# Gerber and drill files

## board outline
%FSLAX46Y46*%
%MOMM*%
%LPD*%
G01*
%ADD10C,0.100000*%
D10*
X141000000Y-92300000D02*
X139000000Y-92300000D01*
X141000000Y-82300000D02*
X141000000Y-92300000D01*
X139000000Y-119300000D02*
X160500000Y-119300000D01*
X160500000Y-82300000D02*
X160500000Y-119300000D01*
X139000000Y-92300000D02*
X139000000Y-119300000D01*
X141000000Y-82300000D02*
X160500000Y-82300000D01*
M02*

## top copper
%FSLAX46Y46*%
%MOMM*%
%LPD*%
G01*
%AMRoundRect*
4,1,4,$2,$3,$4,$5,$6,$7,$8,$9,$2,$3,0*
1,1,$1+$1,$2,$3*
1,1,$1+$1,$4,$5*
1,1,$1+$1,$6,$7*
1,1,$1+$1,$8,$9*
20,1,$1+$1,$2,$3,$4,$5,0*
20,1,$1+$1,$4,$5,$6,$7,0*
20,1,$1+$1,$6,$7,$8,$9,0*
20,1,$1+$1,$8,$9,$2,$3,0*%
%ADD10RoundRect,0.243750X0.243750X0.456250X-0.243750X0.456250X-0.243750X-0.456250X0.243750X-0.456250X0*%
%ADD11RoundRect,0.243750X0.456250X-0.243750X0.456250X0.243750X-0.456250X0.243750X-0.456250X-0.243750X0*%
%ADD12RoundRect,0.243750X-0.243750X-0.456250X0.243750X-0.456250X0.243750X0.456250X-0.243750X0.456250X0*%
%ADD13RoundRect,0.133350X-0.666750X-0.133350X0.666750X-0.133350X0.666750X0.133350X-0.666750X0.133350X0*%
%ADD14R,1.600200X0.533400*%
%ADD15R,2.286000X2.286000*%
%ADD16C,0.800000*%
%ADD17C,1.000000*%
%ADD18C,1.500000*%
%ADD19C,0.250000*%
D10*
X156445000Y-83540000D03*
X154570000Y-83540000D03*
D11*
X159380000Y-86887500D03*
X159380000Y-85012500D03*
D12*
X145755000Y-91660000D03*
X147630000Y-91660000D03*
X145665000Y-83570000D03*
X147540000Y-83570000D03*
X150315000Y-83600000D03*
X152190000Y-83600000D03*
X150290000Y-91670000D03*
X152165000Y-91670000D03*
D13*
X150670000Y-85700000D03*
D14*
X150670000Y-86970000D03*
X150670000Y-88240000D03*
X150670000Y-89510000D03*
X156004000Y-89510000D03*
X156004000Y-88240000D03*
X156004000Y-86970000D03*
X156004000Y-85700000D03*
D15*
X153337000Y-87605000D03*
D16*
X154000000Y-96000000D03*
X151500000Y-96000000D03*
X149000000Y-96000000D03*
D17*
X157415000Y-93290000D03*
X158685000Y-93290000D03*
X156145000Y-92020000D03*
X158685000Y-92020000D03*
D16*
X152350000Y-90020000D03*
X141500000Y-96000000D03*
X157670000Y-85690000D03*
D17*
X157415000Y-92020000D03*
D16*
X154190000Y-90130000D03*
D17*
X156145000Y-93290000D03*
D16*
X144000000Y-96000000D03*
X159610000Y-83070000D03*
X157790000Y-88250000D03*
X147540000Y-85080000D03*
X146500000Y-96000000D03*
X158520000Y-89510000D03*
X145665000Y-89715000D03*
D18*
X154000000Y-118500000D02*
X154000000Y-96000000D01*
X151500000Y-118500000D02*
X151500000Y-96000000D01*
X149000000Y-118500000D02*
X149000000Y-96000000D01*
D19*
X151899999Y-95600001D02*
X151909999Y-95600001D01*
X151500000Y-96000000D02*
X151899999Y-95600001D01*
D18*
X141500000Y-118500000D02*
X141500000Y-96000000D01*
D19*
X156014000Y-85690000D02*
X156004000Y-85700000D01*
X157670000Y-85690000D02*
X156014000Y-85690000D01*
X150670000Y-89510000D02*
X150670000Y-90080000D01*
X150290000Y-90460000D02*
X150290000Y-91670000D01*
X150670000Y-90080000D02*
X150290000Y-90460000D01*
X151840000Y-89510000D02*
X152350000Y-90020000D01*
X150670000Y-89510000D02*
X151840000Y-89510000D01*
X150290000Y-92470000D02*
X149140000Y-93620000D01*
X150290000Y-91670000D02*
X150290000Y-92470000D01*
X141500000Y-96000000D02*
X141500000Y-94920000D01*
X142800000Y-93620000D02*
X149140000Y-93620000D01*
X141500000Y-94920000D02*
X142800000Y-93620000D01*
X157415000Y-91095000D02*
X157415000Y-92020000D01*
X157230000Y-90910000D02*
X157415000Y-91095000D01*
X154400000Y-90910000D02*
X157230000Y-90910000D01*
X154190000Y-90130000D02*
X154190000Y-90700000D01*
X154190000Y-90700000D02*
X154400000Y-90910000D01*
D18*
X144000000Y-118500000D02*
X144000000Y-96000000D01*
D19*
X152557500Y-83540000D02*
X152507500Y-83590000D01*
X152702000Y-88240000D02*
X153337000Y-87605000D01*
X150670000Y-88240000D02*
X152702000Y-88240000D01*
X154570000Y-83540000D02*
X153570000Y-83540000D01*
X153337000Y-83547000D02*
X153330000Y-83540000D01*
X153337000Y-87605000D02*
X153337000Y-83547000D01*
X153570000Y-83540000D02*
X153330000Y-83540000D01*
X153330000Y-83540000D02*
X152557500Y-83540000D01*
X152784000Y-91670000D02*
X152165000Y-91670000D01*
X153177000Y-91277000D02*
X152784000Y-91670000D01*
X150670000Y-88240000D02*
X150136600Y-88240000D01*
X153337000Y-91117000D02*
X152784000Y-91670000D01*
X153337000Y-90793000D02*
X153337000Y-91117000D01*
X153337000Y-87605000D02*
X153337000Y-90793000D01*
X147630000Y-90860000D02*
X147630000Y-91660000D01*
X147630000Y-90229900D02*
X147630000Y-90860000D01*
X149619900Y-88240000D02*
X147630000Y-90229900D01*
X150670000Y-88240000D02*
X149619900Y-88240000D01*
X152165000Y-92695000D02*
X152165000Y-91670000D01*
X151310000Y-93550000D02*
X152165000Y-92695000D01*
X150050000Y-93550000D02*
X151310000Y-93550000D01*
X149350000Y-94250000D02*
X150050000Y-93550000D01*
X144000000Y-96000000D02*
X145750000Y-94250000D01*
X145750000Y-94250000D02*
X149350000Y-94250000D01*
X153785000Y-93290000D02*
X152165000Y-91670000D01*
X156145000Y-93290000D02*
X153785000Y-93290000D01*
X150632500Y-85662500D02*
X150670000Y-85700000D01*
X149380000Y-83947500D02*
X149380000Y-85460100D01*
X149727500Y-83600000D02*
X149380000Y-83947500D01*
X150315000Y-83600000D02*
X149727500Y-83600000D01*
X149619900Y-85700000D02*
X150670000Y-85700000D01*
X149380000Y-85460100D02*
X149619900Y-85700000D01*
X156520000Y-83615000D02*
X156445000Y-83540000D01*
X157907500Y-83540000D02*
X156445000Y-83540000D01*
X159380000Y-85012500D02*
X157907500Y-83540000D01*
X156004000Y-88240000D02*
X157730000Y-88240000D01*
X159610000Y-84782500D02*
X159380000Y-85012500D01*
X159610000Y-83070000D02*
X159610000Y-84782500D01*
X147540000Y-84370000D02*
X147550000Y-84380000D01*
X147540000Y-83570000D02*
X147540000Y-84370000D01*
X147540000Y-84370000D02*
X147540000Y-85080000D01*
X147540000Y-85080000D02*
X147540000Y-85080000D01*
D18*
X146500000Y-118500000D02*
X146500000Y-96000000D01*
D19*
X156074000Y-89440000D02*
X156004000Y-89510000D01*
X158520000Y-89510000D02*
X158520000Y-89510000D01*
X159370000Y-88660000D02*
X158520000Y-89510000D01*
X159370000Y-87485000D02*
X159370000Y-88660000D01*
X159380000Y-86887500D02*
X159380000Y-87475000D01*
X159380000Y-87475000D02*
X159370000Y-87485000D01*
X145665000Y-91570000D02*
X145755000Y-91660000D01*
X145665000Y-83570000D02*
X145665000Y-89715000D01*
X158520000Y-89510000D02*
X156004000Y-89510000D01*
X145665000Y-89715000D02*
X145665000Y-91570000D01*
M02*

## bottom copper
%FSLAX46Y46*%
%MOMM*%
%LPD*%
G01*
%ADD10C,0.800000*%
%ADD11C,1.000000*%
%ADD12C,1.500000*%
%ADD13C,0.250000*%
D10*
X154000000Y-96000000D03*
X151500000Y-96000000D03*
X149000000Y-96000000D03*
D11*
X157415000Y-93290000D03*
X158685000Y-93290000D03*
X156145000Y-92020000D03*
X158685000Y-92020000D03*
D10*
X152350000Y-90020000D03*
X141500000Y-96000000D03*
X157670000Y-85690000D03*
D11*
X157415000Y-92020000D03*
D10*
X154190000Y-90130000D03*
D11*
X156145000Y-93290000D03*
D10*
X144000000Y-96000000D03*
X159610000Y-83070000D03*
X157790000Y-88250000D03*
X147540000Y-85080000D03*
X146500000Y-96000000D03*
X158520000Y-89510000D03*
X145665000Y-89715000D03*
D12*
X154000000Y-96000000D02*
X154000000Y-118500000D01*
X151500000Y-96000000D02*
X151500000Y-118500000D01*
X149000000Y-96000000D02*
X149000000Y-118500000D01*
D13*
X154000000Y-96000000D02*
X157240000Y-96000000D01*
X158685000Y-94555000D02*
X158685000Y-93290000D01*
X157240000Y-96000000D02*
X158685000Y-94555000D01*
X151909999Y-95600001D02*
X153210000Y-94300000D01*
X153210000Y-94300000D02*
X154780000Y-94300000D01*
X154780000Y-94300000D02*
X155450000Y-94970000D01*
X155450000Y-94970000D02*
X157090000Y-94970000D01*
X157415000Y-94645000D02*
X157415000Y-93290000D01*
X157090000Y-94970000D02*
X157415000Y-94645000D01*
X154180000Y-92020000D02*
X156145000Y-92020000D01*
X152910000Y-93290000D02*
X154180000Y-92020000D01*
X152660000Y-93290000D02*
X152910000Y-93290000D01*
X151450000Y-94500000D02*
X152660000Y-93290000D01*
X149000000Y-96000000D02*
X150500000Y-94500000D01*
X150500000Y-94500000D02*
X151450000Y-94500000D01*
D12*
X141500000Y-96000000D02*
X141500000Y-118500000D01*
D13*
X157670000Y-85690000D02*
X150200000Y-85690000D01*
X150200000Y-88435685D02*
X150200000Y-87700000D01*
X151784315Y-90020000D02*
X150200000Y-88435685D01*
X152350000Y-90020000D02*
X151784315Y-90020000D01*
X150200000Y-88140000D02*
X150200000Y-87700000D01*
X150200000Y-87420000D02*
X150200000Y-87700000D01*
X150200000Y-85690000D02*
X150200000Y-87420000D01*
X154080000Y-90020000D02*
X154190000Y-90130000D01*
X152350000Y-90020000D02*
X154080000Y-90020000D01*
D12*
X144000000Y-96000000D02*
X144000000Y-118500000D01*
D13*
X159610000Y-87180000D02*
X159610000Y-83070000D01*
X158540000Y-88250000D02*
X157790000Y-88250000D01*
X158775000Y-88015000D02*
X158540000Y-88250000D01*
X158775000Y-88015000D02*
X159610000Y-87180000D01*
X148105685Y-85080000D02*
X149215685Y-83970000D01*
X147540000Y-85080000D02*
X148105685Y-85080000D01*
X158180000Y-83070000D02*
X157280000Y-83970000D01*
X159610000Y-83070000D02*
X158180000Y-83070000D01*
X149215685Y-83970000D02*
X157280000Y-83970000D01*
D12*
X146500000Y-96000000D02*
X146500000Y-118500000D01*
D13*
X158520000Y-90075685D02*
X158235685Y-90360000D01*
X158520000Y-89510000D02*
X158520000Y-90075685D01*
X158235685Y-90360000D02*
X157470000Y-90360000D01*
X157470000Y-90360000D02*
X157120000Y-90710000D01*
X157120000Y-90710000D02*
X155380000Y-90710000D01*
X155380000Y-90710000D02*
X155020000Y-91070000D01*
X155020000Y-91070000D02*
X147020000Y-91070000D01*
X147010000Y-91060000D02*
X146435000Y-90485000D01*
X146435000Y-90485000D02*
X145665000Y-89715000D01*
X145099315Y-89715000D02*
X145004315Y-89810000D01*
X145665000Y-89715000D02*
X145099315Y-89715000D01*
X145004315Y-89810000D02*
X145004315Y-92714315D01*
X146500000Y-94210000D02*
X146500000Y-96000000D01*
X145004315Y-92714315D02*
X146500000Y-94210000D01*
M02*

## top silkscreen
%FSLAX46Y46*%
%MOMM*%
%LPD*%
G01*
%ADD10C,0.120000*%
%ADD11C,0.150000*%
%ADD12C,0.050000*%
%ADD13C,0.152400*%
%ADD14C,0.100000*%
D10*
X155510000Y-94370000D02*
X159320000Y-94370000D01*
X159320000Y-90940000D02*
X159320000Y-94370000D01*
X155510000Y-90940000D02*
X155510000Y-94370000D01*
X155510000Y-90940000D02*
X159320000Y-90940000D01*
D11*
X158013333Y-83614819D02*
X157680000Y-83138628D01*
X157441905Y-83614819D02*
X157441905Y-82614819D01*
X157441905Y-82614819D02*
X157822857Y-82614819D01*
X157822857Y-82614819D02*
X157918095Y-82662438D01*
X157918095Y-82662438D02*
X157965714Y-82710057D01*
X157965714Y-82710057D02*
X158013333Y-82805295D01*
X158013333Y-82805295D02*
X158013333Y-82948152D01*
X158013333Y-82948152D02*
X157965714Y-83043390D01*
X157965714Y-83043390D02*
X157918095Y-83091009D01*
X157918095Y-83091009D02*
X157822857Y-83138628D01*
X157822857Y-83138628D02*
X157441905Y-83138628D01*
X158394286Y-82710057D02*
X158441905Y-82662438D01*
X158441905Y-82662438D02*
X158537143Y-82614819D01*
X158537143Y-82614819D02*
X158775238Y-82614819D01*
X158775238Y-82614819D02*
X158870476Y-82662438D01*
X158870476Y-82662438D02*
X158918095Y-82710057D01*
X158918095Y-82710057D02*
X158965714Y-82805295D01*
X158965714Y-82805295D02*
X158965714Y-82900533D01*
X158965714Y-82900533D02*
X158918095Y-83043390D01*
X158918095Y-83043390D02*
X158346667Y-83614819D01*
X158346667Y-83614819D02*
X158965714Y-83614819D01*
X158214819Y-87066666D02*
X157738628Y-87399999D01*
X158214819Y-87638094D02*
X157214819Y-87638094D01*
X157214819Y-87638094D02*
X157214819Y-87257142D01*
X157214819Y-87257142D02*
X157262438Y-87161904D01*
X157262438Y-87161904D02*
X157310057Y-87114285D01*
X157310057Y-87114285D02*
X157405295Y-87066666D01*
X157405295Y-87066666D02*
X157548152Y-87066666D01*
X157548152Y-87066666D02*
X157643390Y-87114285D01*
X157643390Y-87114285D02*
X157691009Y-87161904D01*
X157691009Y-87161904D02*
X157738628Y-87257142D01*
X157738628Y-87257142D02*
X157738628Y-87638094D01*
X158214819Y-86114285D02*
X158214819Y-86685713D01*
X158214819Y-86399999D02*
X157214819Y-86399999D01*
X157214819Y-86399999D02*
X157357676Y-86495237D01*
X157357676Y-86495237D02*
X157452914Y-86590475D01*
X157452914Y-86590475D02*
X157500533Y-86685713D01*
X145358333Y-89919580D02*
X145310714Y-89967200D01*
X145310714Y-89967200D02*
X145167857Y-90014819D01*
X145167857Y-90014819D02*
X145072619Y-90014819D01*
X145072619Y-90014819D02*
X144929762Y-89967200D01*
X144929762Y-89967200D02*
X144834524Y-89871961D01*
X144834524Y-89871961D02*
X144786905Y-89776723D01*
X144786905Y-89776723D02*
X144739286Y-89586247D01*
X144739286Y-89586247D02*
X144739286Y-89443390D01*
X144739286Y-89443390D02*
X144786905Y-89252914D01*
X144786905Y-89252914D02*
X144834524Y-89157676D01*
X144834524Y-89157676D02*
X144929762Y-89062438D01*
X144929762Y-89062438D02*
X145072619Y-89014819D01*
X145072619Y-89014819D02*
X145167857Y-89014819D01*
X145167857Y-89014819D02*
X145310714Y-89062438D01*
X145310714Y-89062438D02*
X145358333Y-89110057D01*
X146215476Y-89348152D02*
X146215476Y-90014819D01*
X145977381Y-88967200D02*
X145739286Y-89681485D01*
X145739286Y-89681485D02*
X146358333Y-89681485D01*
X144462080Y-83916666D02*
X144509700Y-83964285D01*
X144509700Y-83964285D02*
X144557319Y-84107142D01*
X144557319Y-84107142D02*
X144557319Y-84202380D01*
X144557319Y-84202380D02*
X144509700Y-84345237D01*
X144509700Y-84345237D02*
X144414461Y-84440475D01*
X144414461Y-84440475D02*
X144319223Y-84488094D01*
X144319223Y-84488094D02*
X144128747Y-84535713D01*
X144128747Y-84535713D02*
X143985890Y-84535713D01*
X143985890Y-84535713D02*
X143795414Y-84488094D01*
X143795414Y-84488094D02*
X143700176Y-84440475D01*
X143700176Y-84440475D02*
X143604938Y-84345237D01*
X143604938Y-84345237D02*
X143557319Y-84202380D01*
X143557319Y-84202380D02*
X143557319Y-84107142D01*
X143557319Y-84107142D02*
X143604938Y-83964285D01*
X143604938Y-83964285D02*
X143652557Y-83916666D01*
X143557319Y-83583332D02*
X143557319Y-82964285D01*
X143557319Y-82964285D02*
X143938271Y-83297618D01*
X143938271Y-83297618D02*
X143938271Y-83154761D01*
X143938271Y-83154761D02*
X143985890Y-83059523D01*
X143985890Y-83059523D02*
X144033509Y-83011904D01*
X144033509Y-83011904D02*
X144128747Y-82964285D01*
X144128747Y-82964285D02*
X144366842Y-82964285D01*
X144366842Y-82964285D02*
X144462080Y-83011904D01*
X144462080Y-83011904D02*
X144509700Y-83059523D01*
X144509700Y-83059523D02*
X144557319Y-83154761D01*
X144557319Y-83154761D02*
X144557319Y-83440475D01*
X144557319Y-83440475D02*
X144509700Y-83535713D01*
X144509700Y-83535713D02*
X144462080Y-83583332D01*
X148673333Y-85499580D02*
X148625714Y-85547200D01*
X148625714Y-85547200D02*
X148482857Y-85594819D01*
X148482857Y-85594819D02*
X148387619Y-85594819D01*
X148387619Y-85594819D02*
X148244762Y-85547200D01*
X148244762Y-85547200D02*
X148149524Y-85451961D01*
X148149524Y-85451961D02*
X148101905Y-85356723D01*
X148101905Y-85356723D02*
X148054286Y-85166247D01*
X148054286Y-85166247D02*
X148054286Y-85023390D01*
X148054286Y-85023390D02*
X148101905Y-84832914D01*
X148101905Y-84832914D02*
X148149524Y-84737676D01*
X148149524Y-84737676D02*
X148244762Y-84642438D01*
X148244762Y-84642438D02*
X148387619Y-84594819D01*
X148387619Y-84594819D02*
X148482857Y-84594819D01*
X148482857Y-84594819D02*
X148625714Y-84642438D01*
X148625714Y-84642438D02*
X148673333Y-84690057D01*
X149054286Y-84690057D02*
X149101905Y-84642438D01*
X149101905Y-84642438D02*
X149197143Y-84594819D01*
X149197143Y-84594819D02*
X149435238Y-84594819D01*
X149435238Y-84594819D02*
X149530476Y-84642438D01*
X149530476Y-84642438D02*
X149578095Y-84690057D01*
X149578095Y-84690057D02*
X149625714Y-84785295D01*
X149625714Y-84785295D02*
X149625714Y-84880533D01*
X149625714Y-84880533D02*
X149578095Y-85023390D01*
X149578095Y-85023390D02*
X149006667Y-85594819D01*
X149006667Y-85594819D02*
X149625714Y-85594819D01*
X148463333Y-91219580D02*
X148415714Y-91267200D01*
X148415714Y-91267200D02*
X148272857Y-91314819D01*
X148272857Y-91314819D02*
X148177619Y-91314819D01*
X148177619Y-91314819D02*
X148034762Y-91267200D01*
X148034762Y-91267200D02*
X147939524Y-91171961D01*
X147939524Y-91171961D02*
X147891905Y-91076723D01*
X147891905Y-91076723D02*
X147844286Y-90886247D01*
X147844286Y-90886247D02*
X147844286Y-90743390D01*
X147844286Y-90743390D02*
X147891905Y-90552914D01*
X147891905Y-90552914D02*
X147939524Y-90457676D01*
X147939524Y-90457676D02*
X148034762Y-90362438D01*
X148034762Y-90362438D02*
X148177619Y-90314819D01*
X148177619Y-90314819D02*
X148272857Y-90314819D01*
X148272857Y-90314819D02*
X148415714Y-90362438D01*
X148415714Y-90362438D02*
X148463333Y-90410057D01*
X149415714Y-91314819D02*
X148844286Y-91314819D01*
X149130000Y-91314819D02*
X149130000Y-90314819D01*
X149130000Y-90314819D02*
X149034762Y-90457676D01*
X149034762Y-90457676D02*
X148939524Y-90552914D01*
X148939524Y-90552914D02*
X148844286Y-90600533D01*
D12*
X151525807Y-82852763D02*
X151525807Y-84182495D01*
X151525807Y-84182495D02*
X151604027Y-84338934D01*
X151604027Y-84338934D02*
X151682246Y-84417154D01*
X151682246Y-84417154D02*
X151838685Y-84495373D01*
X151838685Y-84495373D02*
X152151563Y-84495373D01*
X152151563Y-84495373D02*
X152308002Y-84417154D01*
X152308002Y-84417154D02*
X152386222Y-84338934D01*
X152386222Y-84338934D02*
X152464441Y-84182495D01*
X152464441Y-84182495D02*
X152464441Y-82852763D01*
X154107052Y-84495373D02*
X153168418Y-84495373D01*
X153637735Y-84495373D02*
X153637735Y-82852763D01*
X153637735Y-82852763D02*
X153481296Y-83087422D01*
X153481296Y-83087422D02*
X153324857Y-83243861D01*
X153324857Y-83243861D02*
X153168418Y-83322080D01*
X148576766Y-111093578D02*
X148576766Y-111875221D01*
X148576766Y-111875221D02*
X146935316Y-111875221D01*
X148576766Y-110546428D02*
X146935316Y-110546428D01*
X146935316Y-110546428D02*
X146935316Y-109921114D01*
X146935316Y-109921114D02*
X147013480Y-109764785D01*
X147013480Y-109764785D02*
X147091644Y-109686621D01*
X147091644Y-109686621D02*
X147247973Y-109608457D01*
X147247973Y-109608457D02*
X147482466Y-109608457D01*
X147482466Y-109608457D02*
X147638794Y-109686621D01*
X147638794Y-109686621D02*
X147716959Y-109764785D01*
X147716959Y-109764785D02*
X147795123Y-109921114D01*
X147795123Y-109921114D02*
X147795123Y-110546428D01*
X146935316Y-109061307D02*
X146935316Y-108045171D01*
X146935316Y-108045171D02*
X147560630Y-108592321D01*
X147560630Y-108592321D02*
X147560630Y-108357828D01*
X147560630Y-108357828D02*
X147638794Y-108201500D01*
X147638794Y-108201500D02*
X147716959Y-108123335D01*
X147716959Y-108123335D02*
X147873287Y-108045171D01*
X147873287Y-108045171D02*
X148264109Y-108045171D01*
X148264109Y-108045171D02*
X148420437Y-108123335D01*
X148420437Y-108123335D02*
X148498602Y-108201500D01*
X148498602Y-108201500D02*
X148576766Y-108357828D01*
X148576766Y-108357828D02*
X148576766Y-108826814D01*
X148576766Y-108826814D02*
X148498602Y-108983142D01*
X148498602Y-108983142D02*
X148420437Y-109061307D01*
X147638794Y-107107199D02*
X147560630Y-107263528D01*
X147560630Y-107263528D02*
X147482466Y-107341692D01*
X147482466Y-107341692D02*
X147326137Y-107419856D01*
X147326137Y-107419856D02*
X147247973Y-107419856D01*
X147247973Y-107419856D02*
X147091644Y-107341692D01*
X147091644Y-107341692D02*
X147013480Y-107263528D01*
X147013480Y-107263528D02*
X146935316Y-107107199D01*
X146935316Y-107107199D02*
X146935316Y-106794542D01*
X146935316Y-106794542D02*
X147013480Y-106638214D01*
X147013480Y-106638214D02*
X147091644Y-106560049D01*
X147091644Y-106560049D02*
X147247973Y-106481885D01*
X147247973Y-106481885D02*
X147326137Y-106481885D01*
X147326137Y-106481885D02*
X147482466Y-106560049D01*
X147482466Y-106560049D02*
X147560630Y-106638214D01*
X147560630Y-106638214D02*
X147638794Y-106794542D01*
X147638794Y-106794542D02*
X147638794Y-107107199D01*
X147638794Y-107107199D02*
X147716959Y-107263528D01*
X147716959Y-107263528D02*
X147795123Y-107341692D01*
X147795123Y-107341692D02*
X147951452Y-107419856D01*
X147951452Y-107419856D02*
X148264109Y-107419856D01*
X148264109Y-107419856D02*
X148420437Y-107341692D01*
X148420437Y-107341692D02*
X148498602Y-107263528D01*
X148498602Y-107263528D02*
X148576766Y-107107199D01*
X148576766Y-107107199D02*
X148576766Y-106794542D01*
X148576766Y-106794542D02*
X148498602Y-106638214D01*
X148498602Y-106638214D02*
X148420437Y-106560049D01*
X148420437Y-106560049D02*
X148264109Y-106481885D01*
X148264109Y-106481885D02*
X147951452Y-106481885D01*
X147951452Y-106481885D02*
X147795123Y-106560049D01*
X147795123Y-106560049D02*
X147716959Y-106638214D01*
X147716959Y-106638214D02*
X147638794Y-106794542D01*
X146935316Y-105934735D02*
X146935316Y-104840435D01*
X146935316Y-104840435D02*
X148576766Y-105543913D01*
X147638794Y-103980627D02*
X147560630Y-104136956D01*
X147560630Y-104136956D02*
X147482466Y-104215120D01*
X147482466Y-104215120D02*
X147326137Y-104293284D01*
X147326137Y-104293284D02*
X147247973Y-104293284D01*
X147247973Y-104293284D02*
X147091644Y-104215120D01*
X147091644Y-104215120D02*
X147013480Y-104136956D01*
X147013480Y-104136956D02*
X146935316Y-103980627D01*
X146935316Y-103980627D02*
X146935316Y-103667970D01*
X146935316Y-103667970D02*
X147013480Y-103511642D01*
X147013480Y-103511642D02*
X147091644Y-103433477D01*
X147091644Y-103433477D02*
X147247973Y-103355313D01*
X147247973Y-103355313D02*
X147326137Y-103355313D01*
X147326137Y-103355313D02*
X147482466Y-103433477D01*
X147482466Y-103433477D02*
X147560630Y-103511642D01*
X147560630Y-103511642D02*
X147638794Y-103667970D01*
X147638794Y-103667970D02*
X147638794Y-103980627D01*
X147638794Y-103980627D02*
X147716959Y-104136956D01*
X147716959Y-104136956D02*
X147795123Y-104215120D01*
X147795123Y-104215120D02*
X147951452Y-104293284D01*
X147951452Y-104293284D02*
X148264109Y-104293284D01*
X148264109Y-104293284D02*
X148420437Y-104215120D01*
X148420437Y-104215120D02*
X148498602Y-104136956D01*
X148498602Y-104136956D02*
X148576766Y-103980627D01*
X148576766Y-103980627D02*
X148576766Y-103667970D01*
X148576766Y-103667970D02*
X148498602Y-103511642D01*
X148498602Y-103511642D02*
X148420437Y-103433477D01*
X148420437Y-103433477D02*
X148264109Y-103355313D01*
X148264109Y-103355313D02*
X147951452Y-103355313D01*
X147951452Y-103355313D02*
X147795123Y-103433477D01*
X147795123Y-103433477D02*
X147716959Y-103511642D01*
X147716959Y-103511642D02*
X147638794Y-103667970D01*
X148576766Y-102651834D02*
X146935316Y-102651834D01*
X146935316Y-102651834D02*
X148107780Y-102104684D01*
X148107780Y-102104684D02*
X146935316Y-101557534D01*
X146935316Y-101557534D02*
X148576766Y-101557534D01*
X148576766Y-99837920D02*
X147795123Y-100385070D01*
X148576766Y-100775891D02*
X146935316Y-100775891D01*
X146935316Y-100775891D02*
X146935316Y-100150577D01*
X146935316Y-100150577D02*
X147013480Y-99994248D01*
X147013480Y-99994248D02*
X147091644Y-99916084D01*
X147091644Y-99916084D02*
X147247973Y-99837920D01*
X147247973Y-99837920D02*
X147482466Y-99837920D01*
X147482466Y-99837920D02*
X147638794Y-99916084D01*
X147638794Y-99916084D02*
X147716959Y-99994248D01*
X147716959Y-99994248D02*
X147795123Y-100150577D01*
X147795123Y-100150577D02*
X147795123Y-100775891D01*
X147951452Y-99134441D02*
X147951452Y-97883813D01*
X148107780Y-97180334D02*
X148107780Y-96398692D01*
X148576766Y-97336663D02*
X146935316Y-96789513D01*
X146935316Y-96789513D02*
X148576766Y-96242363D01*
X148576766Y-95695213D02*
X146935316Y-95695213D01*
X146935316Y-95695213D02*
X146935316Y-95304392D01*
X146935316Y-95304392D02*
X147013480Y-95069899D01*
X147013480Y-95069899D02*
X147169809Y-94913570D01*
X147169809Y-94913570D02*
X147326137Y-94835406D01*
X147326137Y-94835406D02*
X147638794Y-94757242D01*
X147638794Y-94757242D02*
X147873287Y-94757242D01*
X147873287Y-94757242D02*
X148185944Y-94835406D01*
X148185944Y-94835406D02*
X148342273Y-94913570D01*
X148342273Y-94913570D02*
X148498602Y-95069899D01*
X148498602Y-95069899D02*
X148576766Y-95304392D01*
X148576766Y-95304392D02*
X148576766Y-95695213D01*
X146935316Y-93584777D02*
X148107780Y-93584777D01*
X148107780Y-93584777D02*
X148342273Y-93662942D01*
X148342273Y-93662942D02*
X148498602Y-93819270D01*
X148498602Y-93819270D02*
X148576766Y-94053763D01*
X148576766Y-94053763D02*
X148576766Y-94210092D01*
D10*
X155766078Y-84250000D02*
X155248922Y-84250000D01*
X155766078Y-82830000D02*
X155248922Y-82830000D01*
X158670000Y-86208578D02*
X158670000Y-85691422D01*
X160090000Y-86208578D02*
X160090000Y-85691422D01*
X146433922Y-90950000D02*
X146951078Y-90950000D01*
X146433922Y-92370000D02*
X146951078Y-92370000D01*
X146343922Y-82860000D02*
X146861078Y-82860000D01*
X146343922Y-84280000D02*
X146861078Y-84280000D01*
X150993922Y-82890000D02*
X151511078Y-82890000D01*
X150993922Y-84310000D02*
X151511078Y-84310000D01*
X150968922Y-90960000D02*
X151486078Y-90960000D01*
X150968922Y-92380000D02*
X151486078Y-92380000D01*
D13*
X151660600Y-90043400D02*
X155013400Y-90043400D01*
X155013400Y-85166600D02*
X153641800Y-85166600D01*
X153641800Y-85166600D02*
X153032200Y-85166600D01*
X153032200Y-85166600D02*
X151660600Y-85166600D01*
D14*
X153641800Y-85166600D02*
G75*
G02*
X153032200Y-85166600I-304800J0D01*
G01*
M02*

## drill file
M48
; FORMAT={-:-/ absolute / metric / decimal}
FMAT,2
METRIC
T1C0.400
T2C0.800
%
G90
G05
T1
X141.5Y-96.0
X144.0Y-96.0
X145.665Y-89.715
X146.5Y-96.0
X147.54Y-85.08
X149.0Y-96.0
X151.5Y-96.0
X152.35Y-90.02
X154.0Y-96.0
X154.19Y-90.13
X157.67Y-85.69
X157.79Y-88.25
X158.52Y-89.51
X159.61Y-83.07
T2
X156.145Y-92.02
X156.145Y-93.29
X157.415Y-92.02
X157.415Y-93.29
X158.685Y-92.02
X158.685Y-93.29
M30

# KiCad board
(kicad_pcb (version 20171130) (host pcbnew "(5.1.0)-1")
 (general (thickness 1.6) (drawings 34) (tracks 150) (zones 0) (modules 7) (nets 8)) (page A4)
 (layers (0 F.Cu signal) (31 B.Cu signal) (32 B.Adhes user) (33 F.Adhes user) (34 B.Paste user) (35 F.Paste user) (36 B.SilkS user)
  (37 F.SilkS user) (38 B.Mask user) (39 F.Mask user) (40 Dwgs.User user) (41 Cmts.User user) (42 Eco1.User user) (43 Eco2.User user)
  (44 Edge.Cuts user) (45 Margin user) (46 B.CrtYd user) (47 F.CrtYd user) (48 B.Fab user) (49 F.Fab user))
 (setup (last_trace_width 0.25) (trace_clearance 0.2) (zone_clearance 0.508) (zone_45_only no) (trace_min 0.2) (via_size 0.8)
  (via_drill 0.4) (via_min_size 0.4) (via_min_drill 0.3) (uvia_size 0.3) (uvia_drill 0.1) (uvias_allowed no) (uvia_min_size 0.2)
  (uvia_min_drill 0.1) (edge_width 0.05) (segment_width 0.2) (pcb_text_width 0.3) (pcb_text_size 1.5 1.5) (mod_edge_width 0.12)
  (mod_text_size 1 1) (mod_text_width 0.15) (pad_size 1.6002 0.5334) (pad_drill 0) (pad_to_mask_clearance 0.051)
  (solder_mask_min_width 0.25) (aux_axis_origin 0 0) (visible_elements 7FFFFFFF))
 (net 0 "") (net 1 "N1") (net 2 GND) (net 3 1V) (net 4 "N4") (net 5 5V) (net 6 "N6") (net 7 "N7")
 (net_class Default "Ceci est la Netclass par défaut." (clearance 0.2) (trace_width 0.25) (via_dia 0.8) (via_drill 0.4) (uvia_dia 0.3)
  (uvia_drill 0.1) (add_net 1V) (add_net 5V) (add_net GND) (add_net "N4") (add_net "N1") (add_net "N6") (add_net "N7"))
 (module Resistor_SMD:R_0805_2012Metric (layer F.Cu) (at 155.5075 83.54 180)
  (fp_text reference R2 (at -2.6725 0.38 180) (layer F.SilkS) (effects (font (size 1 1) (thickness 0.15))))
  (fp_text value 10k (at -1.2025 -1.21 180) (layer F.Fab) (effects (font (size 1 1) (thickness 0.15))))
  (fp_line (start -0.258578 -0.71) (end 0.258578 -0.71) (layer F.SilkS) (width 0.12))
  (fp_line (start -0.258578 0.71) (end 0.258578 0.71) (layer F.SilkS) (width 0.12))
  (pad 1 smd roundrect (at -0.9375 0 180) (size 0.975 1.4) (layers F.Cu F.Paste F.Mask) (roundrect_rratio 0.25) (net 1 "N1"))
  (pad 2 smd roundrect (at 0.9375 0 180) (size 0.975 1.4) (layers F.Cu F.Paste F.Mask) (roundrect_rratio 0.25) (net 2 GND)))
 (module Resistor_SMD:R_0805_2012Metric (layer F.Cu) (at 159.38 85.95 90)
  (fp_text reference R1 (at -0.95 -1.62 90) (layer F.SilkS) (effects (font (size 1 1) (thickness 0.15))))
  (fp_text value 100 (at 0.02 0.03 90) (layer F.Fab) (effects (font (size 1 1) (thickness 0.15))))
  (fp_line (start -0.258578 -0.71) (end 0.258578 -0.71) (layer F.SilkS) (width 0.12))
  (fp_line (start -0.258578 0.71) (end 0.258578 0.71) (layer F.SilkS) (width 0.12))
  (pad 1 smd roundrect (at -0.9375 0 90) (size 0.975 1.4) (layers F.Cu F.Paste F.Mask) (roundrect_rratio 0.25) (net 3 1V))
  (pad 2 smd roundrect (at 0.9375 0 90) (size 0.975 1.4) (layers F.Cu F.Paste F.Mask) (roundrect_rratio 0.25) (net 1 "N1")))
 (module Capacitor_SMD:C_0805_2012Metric (layer F.Cu) (at 146.6925 91.66)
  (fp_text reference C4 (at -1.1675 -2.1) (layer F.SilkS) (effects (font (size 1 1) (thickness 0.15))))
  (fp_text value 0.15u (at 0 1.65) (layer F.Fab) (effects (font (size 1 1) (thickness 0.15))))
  (fp_line (start -0.258578 -0.71) (end 0.258578 -0.71) (layer F.SilkS) (width 0.12))
  (fp_line (start -0.258578 0.71) (end 0.258578 0.71) (layer F.SilkS) (width 0.12))
  (pad 1 smd roundrect (at -0.9375 0) (size 0.975 1.4) (layers F.Cu F.Paste F.Mask) (roundrect_rratio 0.25) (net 3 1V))
  (pad 2 smd roundrect (at 0.9375 0) (size 0.975 1.4) (layers F.Cu F.Paste F.Mask) (roundrect_rratio 0.25) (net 2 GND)))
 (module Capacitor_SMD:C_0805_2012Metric (layer F.Cu) (at 146.6025 83.57)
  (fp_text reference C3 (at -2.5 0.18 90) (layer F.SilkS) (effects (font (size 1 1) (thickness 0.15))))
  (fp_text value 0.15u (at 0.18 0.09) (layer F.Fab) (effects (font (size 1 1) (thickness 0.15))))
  (fp_line (start -0.258578 -0.71) (end 0.258578 -0.71) (layer F.SilkS) (width 0.12))
  (fp_line (start -0.258578 0.71) (end 0.258578 0.71) (layer F.SilkS) (width 0.12))
  (pad 1 smd roundrect (at -0.9375 0) (size 0.975 1.4) (layers F.Cu F.Paste F.Mask) (roundrect_rratio 0.25) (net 3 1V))
  (pad 2 smd roundrect (at 0.9375 0) (size 0.975 1.4) (layers F.Cu F.Paste F.Mask) (roundrect_rratio 0.25) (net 1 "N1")))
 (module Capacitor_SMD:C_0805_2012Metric (layer F.Cu) (at 151.2525 83.6)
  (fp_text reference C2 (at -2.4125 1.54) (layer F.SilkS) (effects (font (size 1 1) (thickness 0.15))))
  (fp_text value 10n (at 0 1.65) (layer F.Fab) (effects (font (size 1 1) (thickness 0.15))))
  (fp_line (start -0.258578 -0.71) (end 0.258578 -0.71) (layer F.SilkS) (width 0.12))
  (fp_line (start -0.258578 0.71) (end 0.258578 0.71) (layer F.SilkS) (width 0.12))
  (pad 1 smd roundrect (at -0.9375 0) (size 0.975 1.4) (layers F.Cu F.Paste F.Mask) (roundrect_rratio 0.25) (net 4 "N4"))
  (pad 2 smd roundrect (at 0.9375 0) (size 0.975 1.4) (layers F.Cu F.Paste F.Mask) (roundrect_rratio 0.25) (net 2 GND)))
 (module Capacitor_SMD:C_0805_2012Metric (layer F.Cu) (at 151.2275 91.67)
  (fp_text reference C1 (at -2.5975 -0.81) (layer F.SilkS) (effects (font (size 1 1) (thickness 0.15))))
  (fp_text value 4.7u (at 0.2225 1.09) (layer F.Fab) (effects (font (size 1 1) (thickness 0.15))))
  (fp_line (start -0.258578 -0.71) (end 0.258578 -0.71) (layer F.SilkS) (width 0.12))
  (fp_line (start -0.258578 0.71) (end 0.258578 0.71) (layer F.SilkS) (width 0.12))
  (pad 1 smd roundrect (at -0.9375 0) (size 0.975 1.4) (layers F.Cu F.Paste F.Mask) (roundrect_rratio 0.25) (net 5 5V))
  (pad 2 smd roundrect (at 0.9375 0) (size 0.975 1.4) (layers F.Cu F.Paste F.Mask) (roundrect_rratio 0.25) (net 2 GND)))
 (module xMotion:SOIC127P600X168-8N (layer F.Cu) (at 153.337 87.605)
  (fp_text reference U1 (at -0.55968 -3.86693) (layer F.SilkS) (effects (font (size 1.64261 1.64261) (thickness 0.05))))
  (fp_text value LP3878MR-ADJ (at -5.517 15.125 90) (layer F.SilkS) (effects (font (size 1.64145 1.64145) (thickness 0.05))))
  (fp_line (start -1.6764 2.4384) (end 1.6764 2.4384) (layer F.SilkS) (width 0.1524))
  (fp_line (start 1.6764 -2.4384) (end 0.3048 -2.4384) (layer F.SilkS) (width 0.1524))
  (fp_line (start 0.3048 -2.4384) (end -0.3048 -2.4384) (layer F.SilkS) (width 0.1524))
  (fp_line (start -0.3048 -2.4384) (end -1.6764 -2.4384) (layer F.SilkS) (width 0.1524))
  (fp_arc (start 0 -2.4384) (end -0.3048 -2.4384) (angle -180) (layer F.SilkS) (width 0.1))
  (pad 1 smd roundrect (at -2.667 -1.905) (size 1.6002 0.5334) (layers F.Cu F.Paste F.Mask) (roundrect_rratio 0.25) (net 4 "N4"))
  (pad 2 smd rect (at -2.667 -0.635) (size 1.6002 0.5334) (layers F.Cu F.Paste F.Mask) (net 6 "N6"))
  (pad 3 smd rect (at -2.667 0.635) (size 1.6002 0.5334) (layers F.Cu F.Paste F.Mask) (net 2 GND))
  (pad 4 smd rect (at -2.667 1.905) (size 1.6002 0.5334) (layers F.Cu F.Paste F.Mask) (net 5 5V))
  (pad 5 smd rect (at 2.667 1.905) (size 1.6002 0.5334) (layers F.Cu F.Paste F.Mask) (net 3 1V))
  (pad 6 smd rect (at 2.667 0.635) (size 1.6002 0.5334) (layers F.Cu F.Paste F.Mask) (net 1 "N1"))
  (pad 7 smd rect (at 2.667 -0.635) (size 1.6002 0.5334) (layers F.Cu F.Paste F.Mask) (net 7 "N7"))
  (pad 8 smd rect (at 2.667 -1.905) (size 1.6002 0.5334) (layers F.Cu F.Paste F.Mask) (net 5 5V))
  (pad 9 smd rect (at 0 0) (size 2.286 2.286) (layers F.Cu F.Paste F.Mask) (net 2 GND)))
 (gr_line (start 155.51 94.37) (end 159.32 94.37) (layer F.SilkS) (width 0.12))
 (gr_line (start 159.32 90.94) (end 159.32 94.37) (layer F.SilkS) (width 0.12))
 (gr_line (start 155.51 90.94) (end 155.51 94.37) (layer F.SilkS) (width 0.12))
 (gr_line (start 155.51 90.94) (end 159.32 90.94) (layer F.SilkS) (width 0.12))
 (gr_line (start 141 92.3) (end 139 92.3) (layer Edge.Cuts) (width 0.1))
 (gr_line (start 141 82.3) (end 141 92.3) (layer Edge.Cuts) (width 0.1))
 (gr_line (start 139 119.3) (end 160.5 119.3) (layer Edge.Cuts) (width 0.1))
 (gr_line (start 160.5 82.3) (end 160.5 119.3) (layer Edge.Cuts) (width 0.1))
 (gr_line (start 139 92.3) (end 139 119.3) (layer Edge.Cuts) (width 0.1))
 (gr_line (start 141 82.3) (end 160.5 82.3) (layer Edge.Cuts) (width 0.1))
 (segment (start 154 118.5) (end 154 96) (width 1.5) (layer F.Cu) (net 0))
 (via (at 154 96) (size 0.8) (drill 0.4) (layers F.Cu B.Cu) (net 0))
 (via (at 151.5 96) (size 0.8) (drill 0.4) (layers F.Cu B.Cu) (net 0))
 (segment (start 154 96) (end 154 118.5) (width 1.5) (layer B.Cu) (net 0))
 (segment (start 151.5 96) (end 151.5 118.5) (width 1.5) (layer B.Cu) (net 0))
 (segment (start 151.5 118.5) (end 151.5 96) (width 1.5) (layer F.Cu) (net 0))
 (via (at 149 96) (size 0.8) (drill 0.4) (layers F.Cu B.Cu) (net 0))
 (segment (start 149 118.5) (end 149 96) (width 1.5) (layer F.Cu) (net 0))
 (segment (start 149 96) (end 149 118.5) (width 1.5) (layer B.Cu) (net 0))
 (via (at 157.415 93.29) (size 1) (drill 0.8) (layers F.Cu B.Cu) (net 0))
 (via (at 158.685 93.29) (size 1) (drill 0.8) (layers F.Cu B.Cu) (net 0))
 (via (at 156.145 92.02) (size 1) (drill 0.8) (layers F.Cu B.Cu) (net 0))
 (via (at 158.685 92.02) (size 1) (drill 0.8) (layers F.Cu B.Cu) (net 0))
 (segment (start 154 96) (end 157.24 96) (width 0.25) (layer B.Cu) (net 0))
 (segment (start 158.685 94.555) (end 158.685 93.29) (width 0.25) (layer B.Cu) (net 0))
 (segment (start 157.24 96) (end 158.685 94.555) (width 0.25) (layer B.Cu) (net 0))
 (segment (start 151.899999 95.600001) (end 151.909999 95.600001) (width 0.25) (layer F.Cu) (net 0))
 (segment (start 151.5 96) (end 151.899999 95.600001) (width 0.25) (layer F.Cu) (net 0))
 (segment (start 151.909999 95.600001) (end 153.21 94.3) (width 0.25) (layer B.Cu) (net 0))
 (segment (start 153.21 94.3) (end 154.78 94.3) (width 0.25) (layer B.Cu) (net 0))
 (segment (start 154.78 94.3) (end 155.45 94.97) (width 0.25) (layer B.Cu) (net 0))
 (segment (start 155.45 94.97) (end 157.09 94.97) (width 0.25) (layer B.Cu) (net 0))
 (segment (start 157.415 94.645) (end 157.415 93.29) (width 0.25) (layer B.Cu) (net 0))
 (segment (start 157.09 94.97) (end 157.415 94.645) (width 0.25) (layer B.Cu) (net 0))
 (segment (start 154.18 92.02) (end 156.145 92.02) (width 0.25) (layer B.Cu) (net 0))
 (segment (start 152.91 93.29) (end 154.18 92.02) (width 0.25) (layer B.Cu) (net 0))
 (segment (start 152.66 93.29) (end 152.91 93.29) (width 0.25) (layer B.Cu) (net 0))
 (segment (start 151.45 94.5) (end 152.66 93.29) (width 0.25) (layer B.Cu) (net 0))
 (segment (start 149 96) (end 150.5 94.5) (width 0.25) (layer B.Cu) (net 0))
 (segment (start 150.5 94.5) (end 151.45 94.5) (width 0.25) (layer B.Cu) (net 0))
 (via (at 152.35 90.02) (size 0.8) (drill 0.4) (layers F.Cu B.Cu) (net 5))
 (via (at 141.5 96) (size 0.8) (drill 0.4) (layers F.Cu B.Cu) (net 5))
 (segment (start 141.5 118.5) (end 141.5 96) (width 1.5) (layer F.Cu) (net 5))
 (segment (start 141.5 96) (end 141.5 118.5) (width 1.5) (layer B.Cu) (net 5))
 (segment (start 156.014 85.69) (end 156.004 85.7) (width 0.25) (layer F.Cu) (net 5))
 (segment (start 157.67 85.69) (end 156.014 85.69) (width 0.25) (layer F.Cu) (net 5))
 (via (at 157.67 85.69) (size 0.8) (drill 0.4) (layers F.Cu B.Cu) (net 5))
 (segment (start 150.67 89.51) (end 150.67 90.08) (width 0.25) (layer F.Cu) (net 5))
 (segment (start 150.29 90.46) (end 150.29 91.67) (width 0.25) (layer F.Cu) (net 5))
 (segment (start 150.67 90.08) (end 150.29 90.46) (width 0.25) (layer F.Cu) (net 5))
 (segment (start 157.67 85.69) (end 150.2 85.69) (width 0.25) (layer B.Cu) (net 5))
 (segment (start 150.2 88.435685) (end 150.2 87.7) (width 0.25) (layer B.Cu) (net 5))
 (segment (start 151.784315 90.02) (end 150.2 88.435685) (width 0.25) (layer B.Cu) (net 5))
 (segment (start 152.35 90.02) (end 151.784315 90.02) (width 0.25) (layer B.Cu) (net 5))
 (segment (start 151.84 89.51) (end 152.35 90.02) (width 0.25) (layer F.Cu) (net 5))
 (segment (start 150.67 89.51) (end 151.84 89.51) (width 0.25) (layer F.Cu) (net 5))
 (segment (start 150.2 88.14) (end 150.2 87.7) (width 0.25) (layer B.Cu) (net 5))
 (segment (start 150.2 87.42) (end 150.2 87.7) (width 0.25) (layer B.Cu) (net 5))
 (segment (start 150.2 85.69) (end 150.2 87.42) (width 0.25) (layer B.Cu) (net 5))
 (via (at 157.415 92.02) (size 1) (drill 0.8) (layers F.Cu B.Cu) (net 5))
 (via (at 154.19 90.13) (size 0.8) (drill 0.4) (layers F.Cu B.Cu) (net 5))
 (segment (start 150.29 92.47) (end 149.14 93.62) (width 0.25) (layer F.Cu) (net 5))
 (segment (start 150.29 91.67) (end 150.29 92.47) (width 0.25) (layer F.Cu) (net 5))
 (segment (start 141.5 96) (end 141.5 94.92) (width 0.25) (layer F.Cu) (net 5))
 (segment (start 142.8 93.62) (end 149.14 93.62) (width 0.25) (layer F.Cu) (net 5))
 (segment (start 141.5 94.92) (end 142.8 93.62) (width 0.25) (layer F.Cu) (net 5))
 (segment (start 154.08 90.02) (end 154.19 90.13) (width 0.25) (layer B.Cu) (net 5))
 (segment (start 152.35 90.02) (end 154.08 90.02) (width 0.25) (layer B.Cu) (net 5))
 (segment (start 157.415 91.095) (end 157.415 92.02) (width 0.25) (layer F.Cu) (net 5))
 (segment (start 157.23 90.91) (end 157.415 91.095) (width 0.25) (layer F.Cu) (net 5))
 (segment (start 154.4 90.91) (end 157.23 90.91) (width 0.25) (layer F.Cu) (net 5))
 (segment (start 154.19 90.13) (end 154.19 90.7) (width 0.25) (layer F.Cu) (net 5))
 (segment (start 154.19 90.7) (end 154.4 90.91) (width 0.25) (layer F.Cu) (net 5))
 (via (at 156.145 93.29) (size 1) (drill 0.8) (layers F.Cu B.Cu) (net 2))
 (via (at 144 96) (size 0.8) (drill 0.4) (layers F.Cu B.Cu) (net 2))
 (segment (start 144 118.5) (end 144 96) (width 1.5) (layer F.Cu) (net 2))
 (segment (start 152.5575 83.54) (end 152.5075 83.59) (width 0.25) (layer F.Cu) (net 2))
 (segment (start 152.702 88.24) (end 153.337 87.605) (width 0.25) (layer F.Cu) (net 2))
 (segment (start 150.67 88.24) (end 152.702 88.24) (width 0.25) (layer F.Cu) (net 2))
 (segment (start 154.57 83.54) (end 153.57 83.54) (width 0.25) (layer F.Cu) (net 2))
 (segment (start 153.337 83.547) (end 153.33 83.54) (width 0.25) (layer F.Cu) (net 2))
 (segment (start 153.337 87.605) (end 153.337 83.547) (width 0.25) (layer F.Cu) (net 2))
 (segment (start 153.57 83.54) (end 153.33 83.54) (width 0.25) (layer F.Cu) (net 2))
 (segment (start 153.33 83.54) (end 152.5575 83.54) (width 0.25) (layer F.Cu) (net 2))
 (segment (start 152.784 91.67) (end 152.165 91.67) (width 0.25) (layer F.Cu) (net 2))
 (segment (start 153.177 91.277) (end 152.784 91.67) (width 0.25) (layer F.Cu) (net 2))
 (segment (start 150.67 88.24) (end 150.1366 88.24) (width 0.25) (layer F.Cu) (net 2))
 (segment (start 144 96) (end 144 118.5) (width 1.5) (layer B.Cu) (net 2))
 (segment (start 153.337 91.117) (end 152.784 91.67) (width 0.25) (layer F.Cu) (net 2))
 (segment (start 153.337 90.793) (end 153.337 91.117) (width 0.25) (layer F.Cu) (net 2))
 (segment (start 153.337 87.605) (end 153.337 90.793) (width 0.25) (layer F.Cu) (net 2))
 (segment (start 147.63 90.86) (end 147.63 91.66) (width 0.25) (layer F.Cu) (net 2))
 (segment (start 147.63 90.2299) (end 147.63 90.86) (width 0.25) (layer F.Cu) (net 2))
 (segment (start 149.6199 88.24) (end 147.63 90.2299) (width 0.25) (layer F.Cu) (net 2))
 (segment (start 150.67 88.24) (end 149.6199 88.24) (width 0.25) (layer F.Cu) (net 2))
 (segment (start 152.165 92.695) (end 152.165 91.67) (width 0.25) (layer F.Cu) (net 2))
 (segment (start 151.31 93.55) (end 152.165 92.695) (width 0.25) (layer F.Cu) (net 2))
 (segment (start 150.05 93.55) (end 151.31 93.55) (width 0.25) (layer F.Cu) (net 2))
 (segment (start 149.35 94.25) (end 150.05 93.55) (width 0.25) (layer F.Cu) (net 2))
 (segment (start 144 96) (end 145.75 94.25) (width 0.25) (layer F.Cu) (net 2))
 (segment (start 145.75 94.25) (end 149.35 94.25) (width 0.25) (layer F.Cu) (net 2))
 (segment (start 153.785 93.29) (end 152.165 91.67) (width 0.25) (layer F.Cu) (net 2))
 (segment (start 156.145 93.29) (end 153.785 93.29) (width 0.25) (layer F.Cu) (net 2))
 (segment (start 150.6325 85.6625) (end 150.67 85.7) (width 0.25) (layer F.Cu) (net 4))
 (segment (start 149.38 83.9475) (end 149.38 85.4601) (width 0.25) (layer F.Cu) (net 4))
 (segment (start 149.7275 83.6) (end 149.38 83.9475) (width 0.25) (layer F.Cu) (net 4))
 (segment (start 150.315 83.6) (end 149.7275 83.6) (width 0.25) (layer F.Cu) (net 4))
 (segment (start 149.6199 85.7) (end 150.67 85.7) (width 0.25) (layer F.Cu) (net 4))
 (segment (start 149.38 85.4601) (end 149.6199 85.7) (width 0.25) (layer F.Cu) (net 4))
 (via (at 159.61 83.07) (size 0.8) (drill 0.4) (layers F.Cu B.Cu) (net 1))
 (segment (start 156.52 83.615) (end 156.445 83.54) (width 0.25) (layer F.Cu) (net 1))
 (segment (start 157.9075 83.54) (end 156.445 83.54) (width 0.25) (layer F.Cu) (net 1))
 (segment (start 159.38 85.0125) (end 157.9075 83.54) (width 0.25) (layer F.Cu) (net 1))
 (via (at 157.79 88.25) (size 0.8) (drill 0.4) (layers F.Cu B.Cu) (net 1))
 (segment (start 156.004 88.24) (end 157.73 88.24) (width 0.25) (layer F.Cu) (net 1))
 (segment (start 159.61 87.18) (end 159.61 83.07) (width 0.25) (layer B.Cu) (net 1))
 (segment (start 159.61 84.7825) (end 159.38 85.0125) (width 0.25) (layer F.Cu) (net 1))
 (segment (start 159.61 83.07) (end 159.61 84.7825) (width 0.25) (layer F.Cu) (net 1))
 (segment (start 158.54 88.25) (end 157.79 88.25) (width 0.25) (layer B.Cu) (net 1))
 (segment (start 158.775 88.015) (end 158.54 88.25) (width 0.25) (layer B.Cu) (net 1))
 (segment (start 158.775 88.015) (end 159.61 87.18) (width 0.25) (layer B.Cu) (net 1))
 (segment (start 147.54 84.37) (end 147.55 84.38) (width 0.25) (layer F.Cu) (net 1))
 (segment (start 147.54 83.57) (end 147.54 84.37) (width 0.25) (layer F.Cu) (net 1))
 (segment (start 147.54 84.37) (end 147.54 85.08) (width 0.25) (layer F.Cu) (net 1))
 (segment (start 147.54 85.08) (end 147.54 85.08) (width 0.25) (layer F.Cu) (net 1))
 (via (at 147.54 85.08) (size 0.8) (drill 0.4) (layers F.Cu B.Cu) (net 1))
 (segment (start 148.105685 85.08) (end 149.215685 83.97) (width 0.25) (layer B.Cu) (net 1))
 (segment (start 147.54 85.08) (end 148.105685 85.08) (width 0.25) (layer B.Cu) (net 1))
 (segment (start 158.18 83.07) (end 157.28 83.97) (width 0.25) (layer B.Cu) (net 1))
 (segment (start 159.61 83.07) (end 158.18 83.07) (width 0.25) (layer B.Cu) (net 1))
 (segment (start 149.215685 83.97) (end 157.28 83.97) (width 0.25) (layer B.Cu) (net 1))
 (via (at 146.5 96) (size 0.8) (drill 0.4) (layers F.Cu B.Cu) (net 3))
 (segment (start 146.5 96) (end 146.5 118.5) (width 1.5) (layer B.Cu) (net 3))
 (segment (start 146.5 118.5) (end 146.5 96) (width 1.5) (layer F.Cu) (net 3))
 (segment (start 156.074 89.44) (end 156.004 89.51) (width 0.25) (layer F.Cu) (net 3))
 (segment (start 158.52 89.51) (end 158.52 89.51) (width 0.25) (layer F.Cu) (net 3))
 (segment (start 159.37 88.66) (end 158.52 89.51) (width 0.25) (layer F.Cu) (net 3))
 (segment (start 159.37 87.485) (end 159.37 88.66) (width 0.25) (layer F.Cu) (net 3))
 (segment (start 159.38 86.8875) (end 159.38 87.475) (width 0.25) (layer F.Cu) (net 3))
 (segment (start 159.38 87.475) (end 159.37 87.485) (width 0.25) (layer F.Cu) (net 3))
 (segment (start 145.665 91.57) (end 145.755 91.66) (width 0.25) (layer F.Cu) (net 3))
 (segment (start 145.665 83.57) (end 145.665 89.715) (width 0.25) (layer F.Cu) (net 3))
 (segment (start 158.52 89.51) (end 156.004 89.51) (width 0.25) (layer F.Cu) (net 3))
 (via (at 158.52 89.51) (size 0.8) (drill 0.4) (layers F.Cu B.Cu) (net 3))
 (segment (start 145.665 89.715) (end 145.665 91.57) (width 0.25) (layer F.Cu) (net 3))
 (via (at 145.665 89.715) (size 0.8) (drill 0.4) (layers F.Cu B.Cu) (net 3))
 (segment (start 158.52 90.075685) (end 158.235685 90.36) (width 0.25) (layer B.Cu) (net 3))
 (segment (start 158.52 89.51) (end 158.52 90.075685) (width 0.25) (layer B.Cu) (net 3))
 (segment (start 158.235685 90.36) (end 157.47 90.36) (width 0.25) (layer B.Cu) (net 3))
 (segment (start 157.47 90.36) (end 157.12 90.71) (width 0.25) (layer B.Cu) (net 3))
 (segment (start 157.12 90.71) (end 155.38 90.71) (width 0.25) (layer B.Cu) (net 3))
 (segment (start 155.38 90.71) (end 155.02 91.07) (width 0.25) (layer B.Cu) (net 3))
 (segment (start 155.02 91.07) (end 147.02 91.07) (width 0.25) (layer B.Cu) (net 3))
 (segment (start 147.01 91.06) (end 146.435 90.485) (width 0.25) (layer B.Cu) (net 3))
 (segment (start 146.435 90.485) (end 145.665 89.715) (width 0.25) (layer B.Cu) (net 3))
 (segment (start 145.099315 89.715) (end 145.004315 89.81) (width 0.25) (layer B.Cu) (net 3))
 (segment (start 145.665 89.715) (end 145.099315 89.715) (width 0.25) (layer B.Cu) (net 3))
 (segment (start 145.004315 89.81) (end 145.004315 92.714315) (width 0.25) (layer B.Cu) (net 3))
 (segment (start 146.5 94.21) (end 146.5 96) (width 0.25) (layer B.Cu) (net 3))
 (segment (start 145.004315 92.714315) (end 146.5 94.21) (width 0.25) (layer B.Cu) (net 3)))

